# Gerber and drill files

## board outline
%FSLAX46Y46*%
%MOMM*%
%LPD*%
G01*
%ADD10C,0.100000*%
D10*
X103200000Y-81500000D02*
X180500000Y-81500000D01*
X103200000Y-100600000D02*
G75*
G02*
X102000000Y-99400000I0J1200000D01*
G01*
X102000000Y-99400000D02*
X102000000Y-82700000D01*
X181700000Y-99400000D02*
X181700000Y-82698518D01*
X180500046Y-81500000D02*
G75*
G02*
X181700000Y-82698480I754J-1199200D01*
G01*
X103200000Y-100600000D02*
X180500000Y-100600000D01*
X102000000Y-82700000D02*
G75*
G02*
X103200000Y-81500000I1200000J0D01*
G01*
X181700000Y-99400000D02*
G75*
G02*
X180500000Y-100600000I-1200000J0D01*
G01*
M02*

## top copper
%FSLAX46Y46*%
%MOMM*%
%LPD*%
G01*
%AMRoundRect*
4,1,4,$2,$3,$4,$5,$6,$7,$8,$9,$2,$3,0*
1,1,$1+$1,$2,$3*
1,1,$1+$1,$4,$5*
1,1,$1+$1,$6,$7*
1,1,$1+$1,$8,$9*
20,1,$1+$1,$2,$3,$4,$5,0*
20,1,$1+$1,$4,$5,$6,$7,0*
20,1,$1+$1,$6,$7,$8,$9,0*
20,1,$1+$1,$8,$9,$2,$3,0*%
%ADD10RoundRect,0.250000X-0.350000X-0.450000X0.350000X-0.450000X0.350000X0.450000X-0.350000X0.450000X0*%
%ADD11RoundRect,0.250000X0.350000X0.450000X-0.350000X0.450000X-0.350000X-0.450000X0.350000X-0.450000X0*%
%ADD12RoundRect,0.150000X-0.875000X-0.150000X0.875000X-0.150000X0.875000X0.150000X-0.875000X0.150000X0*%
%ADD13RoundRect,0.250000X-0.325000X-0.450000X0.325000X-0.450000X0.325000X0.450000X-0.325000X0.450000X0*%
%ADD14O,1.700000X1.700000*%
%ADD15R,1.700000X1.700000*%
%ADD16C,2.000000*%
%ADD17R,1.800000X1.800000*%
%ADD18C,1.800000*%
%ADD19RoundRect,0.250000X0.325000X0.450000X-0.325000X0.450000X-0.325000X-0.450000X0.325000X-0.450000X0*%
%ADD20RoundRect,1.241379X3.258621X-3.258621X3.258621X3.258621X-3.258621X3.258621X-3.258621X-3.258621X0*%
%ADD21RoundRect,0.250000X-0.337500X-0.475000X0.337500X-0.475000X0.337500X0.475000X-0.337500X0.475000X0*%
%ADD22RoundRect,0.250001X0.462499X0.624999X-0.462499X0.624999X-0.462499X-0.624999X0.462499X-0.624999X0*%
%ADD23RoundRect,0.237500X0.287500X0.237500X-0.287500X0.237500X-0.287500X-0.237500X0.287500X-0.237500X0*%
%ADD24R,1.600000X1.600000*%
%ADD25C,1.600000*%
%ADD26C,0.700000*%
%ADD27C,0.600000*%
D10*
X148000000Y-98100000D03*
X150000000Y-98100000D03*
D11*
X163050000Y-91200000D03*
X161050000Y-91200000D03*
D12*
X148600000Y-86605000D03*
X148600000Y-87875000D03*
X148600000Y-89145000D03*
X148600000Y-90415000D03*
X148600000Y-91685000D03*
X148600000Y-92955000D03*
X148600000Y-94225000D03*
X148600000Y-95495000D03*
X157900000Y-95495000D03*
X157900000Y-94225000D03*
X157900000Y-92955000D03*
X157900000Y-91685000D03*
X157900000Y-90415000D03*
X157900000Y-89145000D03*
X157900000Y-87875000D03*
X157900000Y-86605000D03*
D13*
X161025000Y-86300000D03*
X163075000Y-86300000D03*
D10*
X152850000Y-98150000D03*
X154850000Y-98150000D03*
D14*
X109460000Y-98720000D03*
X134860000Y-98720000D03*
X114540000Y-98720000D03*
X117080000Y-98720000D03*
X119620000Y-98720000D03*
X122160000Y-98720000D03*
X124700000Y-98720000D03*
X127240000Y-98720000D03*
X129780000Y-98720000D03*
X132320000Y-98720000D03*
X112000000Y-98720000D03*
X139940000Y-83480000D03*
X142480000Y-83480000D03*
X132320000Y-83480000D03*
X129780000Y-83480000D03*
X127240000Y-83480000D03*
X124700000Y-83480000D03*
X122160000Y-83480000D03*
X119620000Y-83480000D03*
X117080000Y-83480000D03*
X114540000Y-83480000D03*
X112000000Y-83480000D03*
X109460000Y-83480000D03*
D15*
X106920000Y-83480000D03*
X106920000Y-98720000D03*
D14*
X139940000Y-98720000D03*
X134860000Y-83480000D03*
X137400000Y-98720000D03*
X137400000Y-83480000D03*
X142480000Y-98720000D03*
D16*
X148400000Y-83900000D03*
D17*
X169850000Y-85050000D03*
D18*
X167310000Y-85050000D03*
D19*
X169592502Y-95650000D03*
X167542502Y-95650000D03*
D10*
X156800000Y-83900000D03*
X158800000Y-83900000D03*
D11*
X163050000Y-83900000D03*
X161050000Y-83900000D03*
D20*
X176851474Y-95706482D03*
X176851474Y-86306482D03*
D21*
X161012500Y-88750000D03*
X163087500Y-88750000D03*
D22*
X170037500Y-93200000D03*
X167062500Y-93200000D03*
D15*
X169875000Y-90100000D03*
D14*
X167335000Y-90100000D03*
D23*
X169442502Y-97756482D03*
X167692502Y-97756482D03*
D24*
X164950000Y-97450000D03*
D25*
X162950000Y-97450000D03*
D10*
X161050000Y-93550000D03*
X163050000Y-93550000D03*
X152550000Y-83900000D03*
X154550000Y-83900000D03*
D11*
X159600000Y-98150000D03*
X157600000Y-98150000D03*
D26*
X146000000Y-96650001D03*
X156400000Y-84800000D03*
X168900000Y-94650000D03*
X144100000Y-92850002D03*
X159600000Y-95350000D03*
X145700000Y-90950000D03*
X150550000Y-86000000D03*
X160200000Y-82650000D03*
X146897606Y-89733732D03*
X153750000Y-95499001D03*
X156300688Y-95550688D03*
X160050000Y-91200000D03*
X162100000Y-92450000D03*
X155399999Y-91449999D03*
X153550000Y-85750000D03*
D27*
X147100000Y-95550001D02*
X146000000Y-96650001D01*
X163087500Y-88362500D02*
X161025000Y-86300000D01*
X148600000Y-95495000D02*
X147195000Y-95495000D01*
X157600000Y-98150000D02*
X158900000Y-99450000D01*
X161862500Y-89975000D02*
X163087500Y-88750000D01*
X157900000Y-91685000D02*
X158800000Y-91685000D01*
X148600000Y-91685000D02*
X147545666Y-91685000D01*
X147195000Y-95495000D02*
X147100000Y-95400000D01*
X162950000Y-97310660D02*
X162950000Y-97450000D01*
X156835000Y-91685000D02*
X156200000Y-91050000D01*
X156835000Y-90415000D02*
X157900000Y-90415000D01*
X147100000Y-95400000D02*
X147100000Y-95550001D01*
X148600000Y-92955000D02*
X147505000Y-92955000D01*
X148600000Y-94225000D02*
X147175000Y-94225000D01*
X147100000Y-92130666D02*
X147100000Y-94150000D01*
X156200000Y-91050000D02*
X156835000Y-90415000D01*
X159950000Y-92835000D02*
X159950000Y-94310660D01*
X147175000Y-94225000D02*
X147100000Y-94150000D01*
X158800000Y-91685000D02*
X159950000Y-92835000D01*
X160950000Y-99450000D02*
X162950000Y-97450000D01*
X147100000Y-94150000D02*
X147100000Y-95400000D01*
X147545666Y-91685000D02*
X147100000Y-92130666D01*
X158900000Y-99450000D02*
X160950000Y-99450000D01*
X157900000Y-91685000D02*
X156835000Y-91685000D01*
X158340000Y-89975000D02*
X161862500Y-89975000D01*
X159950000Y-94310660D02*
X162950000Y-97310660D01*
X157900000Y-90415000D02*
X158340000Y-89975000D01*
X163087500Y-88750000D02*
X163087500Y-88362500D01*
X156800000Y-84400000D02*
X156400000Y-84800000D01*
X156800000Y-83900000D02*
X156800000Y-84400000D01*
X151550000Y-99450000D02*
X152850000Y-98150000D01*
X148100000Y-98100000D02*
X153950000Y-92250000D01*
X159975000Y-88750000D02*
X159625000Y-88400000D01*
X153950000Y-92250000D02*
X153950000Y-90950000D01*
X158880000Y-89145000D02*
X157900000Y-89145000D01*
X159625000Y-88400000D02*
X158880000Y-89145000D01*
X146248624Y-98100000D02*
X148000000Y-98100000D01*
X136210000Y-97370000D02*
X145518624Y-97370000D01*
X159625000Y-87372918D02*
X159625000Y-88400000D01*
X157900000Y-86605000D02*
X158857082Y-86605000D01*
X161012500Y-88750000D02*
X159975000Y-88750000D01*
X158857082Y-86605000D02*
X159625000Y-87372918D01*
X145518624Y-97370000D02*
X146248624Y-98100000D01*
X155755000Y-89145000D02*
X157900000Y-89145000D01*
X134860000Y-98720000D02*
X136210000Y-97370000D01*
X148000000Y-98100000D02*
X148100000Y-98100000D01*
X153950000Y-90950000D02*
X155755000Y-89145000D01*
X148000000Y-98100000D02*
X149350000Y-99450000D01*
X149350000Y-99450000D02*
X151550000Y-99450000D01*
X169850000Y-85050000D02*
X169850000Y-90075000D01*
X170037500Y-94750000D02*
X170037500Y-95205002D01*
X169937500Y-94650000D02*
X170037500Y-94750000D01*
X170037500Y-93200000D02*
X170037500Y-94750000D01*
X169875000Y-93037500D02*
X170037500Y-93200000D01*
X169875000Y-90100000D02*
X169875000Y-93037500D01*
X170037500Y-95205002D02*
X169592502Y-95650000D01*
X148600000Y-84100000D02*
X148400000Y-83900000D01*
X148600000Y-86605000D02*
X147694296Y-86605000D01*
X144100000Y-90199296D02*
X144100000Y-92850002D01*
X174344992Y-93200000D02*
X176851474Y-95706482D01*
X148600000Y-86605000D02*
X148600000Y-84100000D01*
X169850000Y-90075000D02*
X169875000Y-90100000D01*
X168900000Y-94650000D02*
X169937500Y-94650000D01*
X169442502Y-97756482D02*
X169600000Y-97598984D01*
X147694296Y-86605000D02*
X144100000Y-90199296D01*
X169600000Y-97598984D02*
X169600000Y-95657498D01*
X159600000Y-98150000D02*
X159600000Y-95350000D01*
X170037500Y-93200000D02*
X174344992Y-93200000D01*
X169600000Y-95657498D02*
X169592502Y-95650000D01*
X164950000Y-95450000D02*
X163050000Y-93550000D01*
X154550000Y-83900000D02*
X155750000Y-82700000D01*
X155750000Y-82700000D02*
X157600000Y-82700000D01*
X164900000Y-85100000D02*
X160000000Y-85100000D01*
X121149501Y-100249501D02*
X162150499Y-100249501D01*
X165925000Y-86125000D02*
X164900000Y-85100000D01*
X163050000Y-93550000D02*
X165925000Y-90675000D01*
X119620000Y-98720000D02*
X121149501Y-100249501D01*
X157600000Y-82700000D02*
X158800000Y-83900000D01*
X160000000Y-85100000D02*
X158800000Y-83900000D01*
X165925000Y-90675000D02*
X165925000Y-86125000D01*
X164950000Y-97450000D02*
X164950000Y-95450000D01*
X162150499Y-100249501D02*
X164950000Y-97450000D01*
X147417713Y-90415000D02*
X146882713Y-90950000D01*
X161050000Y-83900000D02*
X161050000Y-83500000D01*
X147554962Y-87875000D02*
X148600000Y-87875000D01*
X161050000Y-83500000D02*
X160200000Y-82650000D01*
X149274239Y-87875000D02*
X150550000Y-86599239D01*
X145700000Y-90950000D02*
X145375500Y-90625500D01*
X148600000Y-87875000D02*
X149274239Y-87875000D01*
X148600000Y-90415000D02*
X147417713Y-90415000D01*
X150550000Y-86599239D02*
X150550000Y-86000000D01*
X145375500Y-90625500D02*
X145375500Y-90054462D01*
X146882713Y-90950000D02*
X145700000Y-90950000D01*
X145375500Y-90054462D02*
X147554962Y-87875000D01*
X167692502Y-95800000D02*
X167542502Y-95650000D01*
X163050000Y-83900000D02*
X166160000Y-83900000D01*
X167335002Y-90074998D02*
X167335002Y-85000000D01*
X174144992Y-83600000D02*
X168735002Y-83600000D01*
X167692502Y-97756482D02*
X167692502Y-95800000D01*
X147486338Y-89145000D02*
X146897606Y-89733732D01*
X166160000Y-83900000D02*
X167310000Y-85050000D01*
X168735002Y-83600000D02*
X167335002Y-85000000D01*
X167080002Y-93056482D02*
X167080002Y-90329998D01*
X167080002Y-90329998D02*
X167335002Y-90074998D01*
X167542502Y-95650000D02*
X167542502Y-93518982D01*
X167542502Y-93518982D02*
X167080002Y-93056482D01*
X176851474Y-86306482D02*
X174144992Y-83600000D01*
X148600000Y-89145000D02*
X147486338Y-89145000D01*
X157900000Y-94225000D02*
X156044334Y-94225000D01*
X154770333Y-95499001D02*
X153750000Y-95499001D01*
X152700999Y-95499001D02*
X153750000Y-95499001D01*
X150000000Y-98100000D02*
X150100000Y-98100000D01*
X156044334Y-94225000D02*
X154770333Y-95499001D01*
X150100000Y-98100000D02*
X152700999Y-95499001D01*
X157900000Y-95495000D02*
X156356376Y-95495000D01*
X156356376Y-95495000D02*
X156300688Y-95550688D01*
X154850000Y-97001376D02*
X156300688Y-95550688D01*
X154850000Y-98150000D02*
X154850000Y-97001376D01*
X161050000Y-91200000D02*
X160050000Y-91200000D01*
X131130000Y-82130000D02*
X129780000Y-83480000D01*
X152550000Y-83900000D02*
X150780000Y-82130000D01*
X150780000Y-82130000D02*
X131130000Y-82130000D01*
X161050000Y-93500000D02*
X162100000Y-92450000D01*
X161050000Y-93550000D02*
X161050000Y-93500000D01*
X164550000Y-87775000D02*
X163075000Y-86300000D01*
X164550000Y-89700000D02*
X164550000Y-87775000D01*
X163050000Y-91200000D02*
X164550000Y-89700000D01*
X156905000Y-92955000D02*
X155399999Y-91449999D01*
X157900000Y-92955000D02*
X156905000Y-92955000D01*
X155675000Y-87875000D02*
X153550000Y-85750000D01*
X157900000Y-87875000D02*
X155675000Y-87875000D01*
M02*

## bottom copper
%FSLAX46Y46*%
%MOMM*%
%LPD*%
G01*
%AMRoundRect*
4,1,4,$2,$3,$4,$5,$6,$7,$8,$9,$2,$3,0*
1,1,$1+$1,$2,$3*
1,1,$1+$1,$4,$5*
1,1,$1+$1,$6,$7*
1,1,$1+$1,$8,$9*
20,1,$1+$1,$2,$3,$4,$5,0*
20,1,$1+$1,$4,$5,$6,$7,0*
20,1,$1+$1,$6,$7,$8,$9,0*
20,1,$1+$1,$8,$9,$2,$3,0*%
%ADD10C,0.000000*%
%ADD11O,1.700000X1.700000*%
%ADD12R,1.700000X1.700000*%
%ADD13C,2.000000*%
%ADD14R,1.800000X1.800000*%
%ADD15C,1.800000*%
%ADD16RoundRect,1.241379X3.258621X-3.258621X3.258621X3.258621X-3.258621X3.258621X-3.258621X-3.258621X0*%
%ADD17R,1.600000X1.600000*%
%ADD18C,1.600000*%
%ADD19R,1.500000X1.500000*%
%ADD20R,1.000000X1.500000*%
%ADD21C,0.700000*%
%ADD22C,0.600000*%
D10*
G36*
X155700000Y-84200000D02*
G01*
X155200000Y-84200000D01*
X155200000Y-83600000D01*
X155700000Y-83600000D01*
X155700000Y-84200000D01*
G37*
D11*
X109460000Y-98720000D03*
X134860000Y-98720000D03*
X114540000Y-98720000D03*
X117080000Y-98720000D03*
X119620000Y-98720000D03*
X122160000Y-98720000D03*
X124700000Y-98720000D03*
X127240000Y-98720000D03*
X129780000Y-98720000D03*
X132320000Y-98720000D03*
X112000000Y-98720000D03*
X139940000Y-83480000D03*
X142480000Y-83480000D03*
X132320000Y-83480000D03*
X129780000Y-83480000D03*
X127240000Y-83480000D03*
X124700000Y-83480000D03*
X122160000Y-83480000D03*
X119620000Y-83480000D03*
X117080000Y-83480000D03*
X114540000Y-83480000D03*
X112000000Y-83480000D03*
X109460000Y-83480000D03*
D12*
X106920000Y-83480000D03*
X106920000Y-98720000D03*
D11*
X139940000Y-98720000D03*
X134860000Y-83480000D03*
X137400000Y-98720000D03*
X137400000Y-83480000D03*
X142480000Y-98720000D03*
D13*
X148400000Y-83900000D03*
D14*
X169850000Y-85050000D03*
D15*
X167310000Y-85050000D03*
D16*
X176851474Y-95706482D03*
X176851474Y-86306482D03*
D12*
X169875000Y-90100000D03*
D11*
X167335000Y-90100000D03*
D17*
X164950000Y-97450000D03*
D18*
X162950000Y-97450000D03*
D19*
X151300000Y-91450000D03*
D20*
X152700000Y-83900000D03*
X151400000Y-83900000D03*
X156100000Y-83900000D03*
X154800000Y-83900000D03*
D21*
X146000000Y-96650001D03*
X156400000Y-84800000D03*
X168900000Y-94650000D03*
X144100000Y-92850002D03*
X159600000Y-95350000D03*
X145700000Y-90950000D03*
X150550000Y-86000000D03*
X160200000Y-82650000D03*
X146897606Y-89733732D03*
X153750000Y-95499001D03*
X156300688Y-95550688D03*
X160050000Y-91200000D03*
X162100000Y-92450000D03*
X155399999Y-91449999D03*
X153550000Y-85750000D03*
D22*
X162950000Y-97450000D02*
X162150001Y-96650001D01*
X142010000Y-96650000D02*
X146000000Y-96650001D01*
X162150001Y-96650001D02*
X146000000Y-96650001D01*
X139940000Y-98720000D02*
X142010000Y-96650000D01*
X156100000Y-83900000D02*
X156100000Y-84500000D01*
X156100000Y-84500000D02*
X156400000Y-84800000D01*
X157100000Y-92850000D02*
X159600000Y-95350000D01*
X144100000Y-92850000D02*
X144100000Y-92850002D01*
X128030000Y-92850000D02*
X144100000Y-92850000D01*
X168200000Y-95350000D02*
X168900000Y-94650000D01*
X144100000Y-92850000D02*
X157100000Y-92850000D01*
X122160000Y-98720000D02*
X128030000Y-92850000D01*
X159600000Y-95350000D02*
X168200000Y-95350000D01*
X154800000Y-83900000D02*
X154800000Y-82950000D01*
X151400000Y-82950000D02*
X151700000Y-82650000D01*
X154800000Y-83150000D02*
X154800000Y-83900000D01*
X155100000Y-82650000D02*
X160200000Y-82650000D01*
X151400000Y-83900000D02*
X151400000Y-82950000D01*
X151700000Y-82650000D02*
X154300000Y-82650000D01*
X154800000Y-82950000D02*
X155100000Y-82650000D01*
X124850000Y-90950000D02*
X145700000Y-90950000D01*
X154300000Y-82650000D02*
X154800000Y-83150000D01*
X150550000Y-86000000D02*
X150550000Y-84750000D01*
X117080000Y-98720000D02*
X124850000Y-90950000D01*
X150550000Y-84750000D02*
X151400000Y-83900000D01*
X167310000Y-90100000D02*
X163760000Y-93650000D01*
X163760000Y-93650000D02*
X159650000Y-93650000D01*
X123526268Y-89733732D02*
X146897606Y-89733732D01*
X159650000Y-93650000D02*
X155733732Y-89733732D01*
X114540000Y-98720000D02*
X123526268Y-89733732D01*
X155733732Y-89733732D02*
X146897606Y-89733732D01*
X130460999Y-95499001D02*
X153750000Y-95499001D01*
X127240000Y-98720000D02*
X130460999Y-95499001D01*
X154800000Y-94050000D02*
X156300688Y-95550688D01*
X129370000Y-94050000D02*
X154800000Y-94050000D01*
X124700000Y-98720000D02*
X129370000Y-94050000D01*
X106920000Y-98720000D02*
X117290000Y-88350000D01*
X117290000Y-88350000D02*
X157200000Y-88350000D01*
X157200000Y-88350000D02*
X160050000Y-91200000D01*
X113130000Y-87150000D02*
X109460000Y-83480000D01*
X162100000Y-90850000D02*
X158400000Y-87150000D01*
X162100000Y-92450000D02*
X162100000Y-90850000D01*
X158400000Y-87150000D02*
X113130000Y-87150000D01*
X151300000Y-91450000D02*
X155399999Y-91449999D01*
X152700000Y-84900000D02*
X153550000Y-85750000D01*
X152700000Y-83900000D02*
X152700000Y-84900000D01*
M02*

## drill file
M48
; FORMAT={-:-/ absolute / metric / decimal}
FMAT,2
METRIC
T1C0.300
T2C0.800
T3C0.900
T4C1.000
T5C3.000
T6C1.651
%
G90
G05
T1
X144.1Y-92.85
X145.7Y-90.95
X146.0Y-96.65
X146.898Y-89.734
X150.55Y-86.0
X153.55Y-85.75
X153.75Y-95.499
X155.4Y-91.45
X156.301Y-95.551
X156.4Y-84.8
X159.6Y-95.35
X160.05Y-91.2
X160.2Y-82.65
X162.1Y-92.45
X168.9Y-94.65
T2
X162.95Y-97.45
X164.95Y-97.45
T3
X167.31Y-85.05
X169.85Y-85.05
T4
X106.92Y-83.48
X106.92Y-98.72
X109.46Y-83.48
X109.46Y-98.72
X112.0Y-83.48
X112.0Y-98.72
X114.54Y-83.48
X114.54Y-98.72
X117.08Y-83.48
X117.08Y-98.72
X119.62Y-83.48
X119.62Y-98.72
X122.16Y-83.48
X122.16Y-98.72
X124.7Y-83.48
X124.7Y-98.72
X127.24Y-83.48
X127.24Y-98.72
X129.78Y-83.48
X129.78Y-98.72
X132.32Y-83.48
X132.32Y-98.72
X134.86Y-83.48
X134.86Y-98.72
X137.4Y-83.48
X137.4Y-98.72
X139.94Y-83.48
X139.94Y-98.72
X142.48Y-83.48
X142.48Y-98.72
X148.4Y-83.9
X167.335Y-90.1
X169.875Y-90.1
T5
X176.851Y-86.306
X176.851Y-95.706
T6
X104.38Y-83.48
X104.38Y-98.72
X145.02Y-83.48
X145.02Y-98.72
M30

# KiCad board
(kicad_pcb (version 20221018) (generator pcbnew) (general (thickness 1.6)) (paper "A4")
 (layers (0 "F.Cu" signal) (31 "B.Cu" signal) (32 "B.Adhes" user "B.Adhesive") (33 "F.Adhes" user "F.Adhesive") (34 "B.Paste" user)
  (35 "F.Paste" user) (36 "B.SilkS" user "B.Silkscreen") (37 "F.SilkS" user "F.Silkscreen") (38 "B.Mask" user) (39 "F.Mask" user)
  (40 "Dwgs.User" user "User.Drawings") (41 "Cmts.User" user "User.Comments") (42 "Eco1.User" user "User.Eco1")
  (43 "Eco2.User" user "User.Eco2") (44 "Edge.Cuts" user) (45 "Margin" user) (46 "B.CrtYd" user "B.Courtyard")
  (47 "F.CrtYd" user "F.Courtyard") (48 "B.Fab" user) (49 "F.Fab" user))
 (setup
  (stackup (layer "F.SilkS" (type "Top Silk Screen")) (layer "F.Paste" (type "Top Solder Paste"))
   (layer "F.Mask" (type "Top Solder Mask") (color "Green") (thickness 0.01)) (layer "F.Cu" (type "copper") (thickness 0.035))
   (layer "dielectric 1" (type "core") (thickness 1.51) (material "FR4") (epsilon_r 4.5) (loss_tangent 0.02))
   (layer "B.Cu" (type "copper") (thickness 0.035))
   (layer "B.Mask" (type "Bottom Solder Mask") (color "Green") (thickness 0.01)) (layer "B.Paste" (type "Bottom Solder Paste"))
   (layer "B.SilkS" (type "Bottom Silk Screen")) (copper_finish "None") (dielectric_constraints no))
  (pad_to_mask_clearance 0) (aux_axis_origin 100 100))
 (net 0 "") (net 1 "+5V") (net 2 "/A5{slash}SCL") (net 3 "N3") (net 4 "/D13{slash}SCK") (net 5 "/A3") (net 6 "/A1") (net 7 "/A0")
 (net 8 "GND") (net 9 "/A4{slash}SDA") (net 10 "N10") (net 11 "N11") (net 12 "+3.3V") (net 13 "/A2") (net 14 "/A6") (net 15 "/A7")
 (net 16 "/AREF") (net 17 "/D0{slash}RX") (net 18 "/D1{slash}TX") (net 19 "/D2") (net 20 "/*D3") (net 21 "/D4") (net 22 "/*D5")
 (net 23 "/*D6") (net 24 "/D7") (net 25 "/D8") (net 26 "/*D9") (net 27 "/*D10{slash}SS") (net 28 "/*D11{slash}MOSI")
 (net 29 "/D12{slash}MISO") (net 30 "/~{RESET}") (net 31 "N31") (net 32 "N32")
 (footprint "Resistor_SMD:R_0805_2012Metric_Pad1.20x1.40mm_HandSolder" (layer "F.Cu") (at 149 98.1)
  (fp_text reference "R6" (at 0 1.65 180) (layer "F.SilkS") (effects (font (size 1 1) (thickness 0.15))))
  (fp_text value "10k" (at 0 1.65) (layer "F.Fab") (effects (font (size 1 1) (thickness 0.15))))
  (pad "1" smd roundrect (at -1 0) (size 1.2 1.4) (layers "F.Cu" "F.Paste" "F.Mask") (roundrect_rratio 0.208333) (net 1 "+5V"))
  (pad "2" smd roundrect (at 1 0) (size 1.2 1.4) (layers "F.Cu" "F.Paste" "F.Mask") (roundrect_rratio 0.208333) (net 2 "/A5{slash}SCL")))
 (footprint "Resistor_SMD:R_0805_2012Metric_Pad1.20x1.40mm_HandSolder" (layer "F.Cu") (at 162.05 91.2 180)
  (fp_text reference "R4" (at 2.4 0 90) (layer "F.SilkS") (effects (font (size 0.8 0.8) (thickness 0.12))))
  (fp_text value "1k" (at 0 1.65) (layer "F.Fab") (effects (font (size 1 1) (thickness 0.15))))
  (pad "1" smd roundrect (at -1 0 180) (size 1.2 1.4) (layers "F.Cu" "F.Paste" "F.Mask") (roundrect_rratio 0.2083333333) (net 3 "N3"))
  (pad "2" smd roundrect (at 1 0 180) (size 1.2 1.4) (layers "F.Cu" "F.Paste" "F.Mask") (roundrect_rratio 0.2083333333)
   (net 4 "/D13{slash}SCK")))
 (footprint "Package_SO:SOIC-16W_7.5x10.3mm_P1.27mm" (layer "F.Cu") (at 153.25 91.05)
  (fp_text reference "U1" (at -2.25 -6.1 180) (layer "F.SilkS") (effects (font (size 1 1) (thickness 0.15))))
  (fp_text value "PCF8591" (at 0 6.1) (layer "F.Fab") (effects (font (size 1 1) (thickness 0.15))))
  (pad "1" smd roundrect (at -4.65 -4.445) (size 2.05 0.6) (layers "F.Cu" "F.Paste" "F.Mask") (roundrect_rratio 0.25) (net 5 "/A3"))
  (pad "2" smd roundrect (at -4.65 -3.175) (size 2.05 0.6) (layers "F.Cu" "F.Paste" "F.Mask") (roundrect_rratio 0.25) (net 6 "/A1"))
  (pad "3" smd roundrect (at -4.65 -1.905) (size 2.05 0.6) (layers "F.Cu" "F.Paste" "F.Mask") (roundrect_rratio 0.25) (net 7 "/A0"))
  (pad "4" smd roundrect (at -4.65 -0.635) (size 2.05 0.6) (layers "F.Cu" "F.Paste" "F.Mask") (roundrect_rratio 0.25) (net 6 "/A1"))
  (pad "5" smd roundrect (at -4.65 0.635) (size 2.05 0.6) (layers "F.Cu" "F.Paste" "F.Mask") (roundrect_rratio 0.25) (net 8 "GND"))
  (pad "6" smd roundrect (at -4.65 1.905) (size 2.05 0.6) (layers "F.Cu" "F.Paste" "F.Mask") (roundrect_rratio 0.25) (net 8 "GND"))
  (pad "7" smd roundrect (at -4.65 3.175) (size 2.05 0.6) (layers "F.Cu" "F.Paste" "F.Mask") (roundrect_rratio 0.25) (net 8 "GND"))
  (pad "8" smd roundrect (at -4.65 4.445) (size 2.05 0.6) (layers "F.Cu" "F.Paste" "F.Mask") (roundrect_rratio 0.25) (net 8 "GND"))
  (pad "9" smd roundrect (at 4.65 4.445) (size 2.05 0.6) (layers "F.Cu" "F.Paste" "F.Mask") (roundrect_rratio 0.25) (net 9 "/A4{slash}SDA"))
  (pad "10" smd roundrect (at 4.65 3.175) (size 2.05 0.6) (layers "F.Cu" "F.Paste" "F.Mask") (roundrect_rratio 0.25) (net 2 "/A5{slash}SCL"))
  (pad "11" smd roundrect (at 4.65 1.905) (size 2.05 0.6) (layers "F.Cu" "F.Paste" "F.Mask") (roundrect_rratio 0.25) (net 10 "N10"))
  (pad "12" smd roundrect (at 4.65 0.635) (size 2.05 0.6) (layers "F.Cu" "F.Paste" "F.Mask") (roundrect_rratio 0.25) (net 8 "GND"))
  (pad "13" smd roundrect (at 4.65 -0.635) (size 2.05 0.6) (layers "F.Cu" "F.Paste" "F.Mask") (roundrect_rratio 0.25) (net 8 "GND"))
  (pad "14" smd roundrect (at 4.65 -1.905) (size 2.05 0.6) (layers "F.Cu" "F.Paste" "F.Mask") (roundrect_rratio 0.25) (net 1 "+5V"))
  (pad "15" smd roundrect (at 4.65 -3.175) (size 2.05 0.6) (layers "F.Cu" "F.Paste" "F.Mask") (roundrect_rratio 0.25) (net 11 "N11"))
  (pad "16" smd roundrect (at 4.65 -4.445) (size 2.05 0.6) (layers "F.Cu" "F.Paste" "F.Mask") (roundrect_rratio 0.25) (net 1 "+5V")))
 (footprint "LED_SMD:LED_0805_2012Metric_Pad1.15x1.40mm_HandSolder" (layer "F.Cu") (at 162.05 86.3)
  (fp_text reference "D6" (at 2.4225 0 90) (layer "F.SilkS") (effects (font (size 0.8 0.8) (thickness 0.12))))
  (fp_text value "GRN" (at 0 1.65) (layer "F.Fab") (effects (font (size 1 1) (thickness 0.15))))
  (pad "1" smd roundrect (at -1.025 0) (size 1.15 1.4) (layers "F.Cu" "F.Paste" "F.Mask") (roundrect_rratio 0.2173913043) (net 8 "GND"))
  (pad "2" smd roundrect (at 1.025 0) (size 1.15 1.4) (layers "F.Cu" "F.Paste" "F.Mask") (roundrect_rratio 0.2173913043) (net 3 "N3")))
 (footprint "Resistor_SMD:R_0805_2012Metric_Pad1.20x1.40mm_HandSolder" (layer "F.Cu") (at 153.85 98.15)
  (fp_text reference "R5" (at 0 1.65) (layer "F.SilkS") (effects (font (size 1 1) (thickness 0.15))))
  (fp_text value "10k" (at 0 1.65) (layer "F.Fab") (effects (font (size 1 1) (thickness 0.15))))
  (pad "1" smd roundrect (at -1 0) (size 1.2 1.4) (layers "F.Cu" "F.Paste" "F.Mask") (roundrect_rratio 0.208333) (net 1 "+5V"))
  (pad "2" smd roundrect (at 1 0) (size 1.2 1.4) (layers "F.Cu" "F.Paste" "F.Mask") (roundrect_rratio 0.208333) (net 9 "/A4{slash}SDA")))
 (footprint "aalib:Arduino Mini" (layer "F.Cu") (at 124.7 91.1 90)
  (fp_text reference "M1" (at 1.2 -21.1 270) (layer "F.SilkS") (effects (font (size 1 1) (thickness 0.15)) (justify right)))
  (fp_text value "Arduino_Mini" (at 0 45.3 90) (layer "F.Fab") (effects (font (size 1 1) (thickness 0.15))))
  (pad "" np_thru_hole circle (at -7.62 -20.32 90) (size 1.651 1.651) (drill 1.651) (layers "*.Mask"))
  (pad "" np_thru_hole circle (at -7.62 20.32 90) (size 1.651 1.651) (drill 1.651) (layers "*.Mask"))
  (pad "" np_thru_hole circle (at 7.62 -20.32 90) (size 1.651 1.651) (drill 1.651) (layers "*.Mask"))
  (pad "" np_thru_hole circle (at 7.62 20.32 90) (size 1.651 1.651) (drill 1.651) (layers "*.Mask"))
  (pad "3V3" thru_hole oval (at -7.62 -15.24 90) (size 1.7 1.7) (drill 1) (layers "*.Cu" "*.Mask") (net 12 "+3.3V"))
  (pad "5V" thru_hole oval (at -7.62 10.16 90) (size 1.7 1.7) (drill 1) (layers "*.Cu" "*.Mask") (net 1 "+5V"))
  (pad "A0" thru_hole oval (at -7.62 -10.16 90) (size 1.7 1.7) (drill 1) (layers "*.Cu" "*.Mask") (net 7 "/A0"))
  (pad "A1" thru_hole oval (at -7.62 -7.62 90) (size 1.7 1.7) (drill 1) (layers "*.Cu" "*.Mask") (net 6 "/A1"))
  (pad "A2" thru_hole oval (at -7.62 -5.08 90) (size 1.7 1.7) (drill 1) (layers "*.Cu" "*.Mask") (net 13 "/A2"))
  (pad "A3" thru_hole oval (at -7.62 -2.54 90) (size 1.7 1.7) (drill 1) (layers "*.Cu" "*.Mask") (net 5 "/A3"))
  (pad "A4" thru_hole oval (at -7.62 0 90) (size 1.7 1.7) (drill 1) (layers "*.Cu" "*.Mask") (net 9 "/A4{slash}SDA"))
  (pad "A5" thru_hole oval (at -7.62 2.54 90) (size 1.7 1.7) (drill 1) (layers "*.Cu" "*.Mask") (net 2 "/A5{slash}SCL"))
  (pad "A6" thru_hole oval (at -7.62 5.08 90) (size 1.7 1.7) (drill 1) (layers "*.Cu" "*.Mask") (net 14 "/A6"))
  (pad "A7" thru_hole oval (at -7.62 7.62 90) (size 1.7 1.7) (drill 1) (layers "*.Cu" "*.Mask") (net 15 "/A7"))
  (pad "AREF" thru_hole oval (at -7.62 -12.7 90) (size 1.7 1.7) (drill 1) (layers "*.Cu" "*.Mask") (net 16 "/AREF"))
  (pad "D0/RX" thru_hole oval (at 7.62 15.24 90) (size 1.7 1.7) (drill 1) (layers "*.Cu" "*.Mask") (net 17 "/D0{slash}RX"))
  (pad "D1/TX" thru_hole oval (at 7.62 17.78 90) (size 1.7 1.7) (drill 1) (layers "*.Cu" "*.Mask") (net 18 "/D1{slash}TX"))
  (pad "D2" thru_hole oval (at 7.62 7.62 90) (size 1.7 1.7) (drill 1) (layers "*.Cu" "*.Mask") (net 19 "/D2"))
  (pad "D3" thru_hole oval (at 7.62 5.08 90) (size 1.7 1.7) (drill 1) (layers "*.Cu" "*.Mask") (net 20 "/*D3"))
  (pad "D4" thru_hole oval (at 7.62 2.54 90) (size 1.7 1.7) (drill 1) (layers "*.Cu" "*.Mask") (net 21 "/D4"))
  (pad "D5" thru_hole oval (at 7.62 0 90) (size 1.7 1.7) (drill 1) (layers "*.Cu" "*.Mask") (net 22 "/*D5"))
  (pad "D6" thru_hole oval (at 7.62 -2.54 90) (size 1.7 1.7) (drill 1) (layers "*.Cu" "*.Mask") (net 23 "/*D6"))
  (pad "D7" thru_hole oval (at 7.62 -5.08 90) (size 1.7 1.7) (drill 1) (layers "*.Cu" "*.Mask") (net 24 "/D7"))
  (pad "D8" thru_hole oval (at 7.62 -7.62 90) (size 1.7 1.7) (drill 1) (layers "*.Cu" "*.Mask") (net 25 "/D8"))
  (pad "D9" thru_hole oval (at 7.62 -10.16 90) (size 1.7 1.7) (drill 1) (layers "*.Cu" "*.Mask") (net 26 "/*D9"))
  (pad "D10" thru_hole oval (at 7.62 -12.7 90) (size 1.7 1.7) (drill 1) (layers "*.Cu" "*.Mask") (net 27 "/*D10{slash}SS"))
  (pad "D11" thru_hole oval (at 7.62 -15.24 90) (size 1.7 1.7) (drill 1) (layers "*.Cu" "*.Mask") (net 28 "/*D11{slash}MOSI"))
  (pad "D12" thru_hole rect (at 7.62 -17.78 90) (size 1.7 1.7) (drill 1) (layers "*.Cu" "*.Mask") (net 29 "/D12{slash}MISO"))
  (pad "D13" thru_hole rect (at -7.62 -17.78 90) (size 1.7 1.7) (drill 1) (layers "*.Cu" "*.Mask") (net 4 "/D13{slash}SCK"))
  (pad "GND" thru_hole oval (at -7.62 15.24 90) (size 1.7 1.7) (drill 1) (layers "*.Cu" "*.Mask") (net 8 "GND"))
  (pad "GND" thru_hole oval (at 7.62 10.16 90) (size 1.7 1.7) (drill 1) (layers "*.Cu" "*.Mask") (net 8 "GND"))
  (pad "RESET" thru_hole oval (at -7.62 12.7 90) (size 1.7 1.7) (drill 1) (layers "*.Cu" "*.Mask") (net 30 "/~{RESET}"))
  (pad "RESET" thru_hole oval (at 7.62 12.7 90) (size 1.7 1.7) (drill 1) (layers "*.Cu" "*.Mask") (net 30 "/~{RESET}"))
  (pad "VIN" thru_hole oval (at -7.62 17.78 90) (size 1.7 1.7) (drill 1) (layers "*.Cu" "*.Mask") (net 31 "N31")))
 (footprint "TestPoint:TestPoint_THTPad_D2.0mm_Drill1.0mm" (layer "F.Cu") (at 148.4 83.9)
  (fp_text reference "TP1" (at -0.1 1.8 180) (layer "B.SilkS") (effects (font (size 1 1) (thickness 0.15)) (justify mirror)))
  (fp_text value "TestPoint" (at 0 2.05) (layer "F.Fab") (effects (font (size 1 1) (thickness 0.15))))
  (pad "1" thru_hole circle (at 0 0) (size 2 2) (drill 1) (layers "*.Cu" "*.Mask") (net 5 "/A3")))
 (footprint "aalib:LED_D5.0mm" (layer "F.Cu") (at 169.85 85.05 180)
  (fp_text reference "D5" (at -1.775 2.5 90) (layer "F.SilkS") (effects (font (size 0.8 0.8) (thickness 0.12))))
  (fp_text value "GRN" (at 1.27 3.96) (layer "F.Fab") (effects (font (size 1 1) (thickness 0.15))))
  (pad "1" thru_hole rect (at 0 0 180) (size 1.8 1.8) (drill 0.9) (layers "*.Cu" "*.Mask") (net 5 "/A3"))
  (pad "2" thru_hole circle (at 2.54 0 180) (size 1.8 1.8) (drill 0.9) (layers "*.Cu" "*.Mask") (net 7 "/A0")))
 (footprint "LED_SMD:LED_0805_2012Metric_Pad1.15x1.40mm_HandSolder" (layer "F.Cu") (at 168.567502 95.65 180)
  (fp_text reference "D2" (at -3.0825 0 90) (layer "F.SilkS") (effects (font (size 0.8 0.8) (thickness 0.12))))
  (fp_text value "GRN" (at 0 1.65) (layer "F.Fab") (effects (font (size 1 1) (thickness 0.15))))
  (pad "1" smd roundrect (at -1.025 0 180) (size 1.15 1.4) (layers "F.Cu" "F.Paste" "F.Mask") (roundrect_rratio 0.217391) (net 5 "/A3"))
  (pad "2" smd roundrect (at 1.025 0 180) (size 1.15 1.4) (layers "F.Cu" "F.Paste" "F.Mask") (roundrect_rratio 0.217391) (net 7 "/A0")))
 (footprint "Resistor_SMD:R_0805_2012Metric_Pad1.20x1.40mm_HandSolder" (layer "F.Cu") (at 157.8 83.9)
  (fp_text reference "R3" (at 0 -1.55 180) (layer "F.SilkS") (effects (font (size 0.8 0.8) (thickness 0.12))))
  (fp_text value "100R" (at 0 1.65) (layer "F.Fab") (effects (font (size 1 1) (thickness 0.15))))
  (pad "1" smd roundrect (at -1 0) (size 1.2 1.4) (layers "F.Cu" "F.Paste" "F.Mask") (roundrect_rratio 0.2083333333) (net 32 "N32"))
  (pad "2" smd roundrect (at 1 0) (size 1.2 1.4) (layers "F.Cu" "F.Paste" "F.Mask") (roundrect_rratio 0.2083333333) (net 13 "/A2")))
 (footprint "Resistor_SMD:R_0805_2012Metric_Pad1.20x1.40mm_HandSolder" (layer "F.Cu") (at 162.05 83.9 180)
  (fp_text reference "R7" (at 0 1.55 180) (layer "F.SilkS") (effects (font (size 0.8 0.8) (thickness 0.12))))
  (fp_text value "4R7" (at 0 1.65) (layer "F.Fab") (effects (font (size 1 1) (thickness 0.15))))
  (pad "1" smd roundrect (at -1 0 180) (size 1.2 1.4) (layers "F.Cu" "F.Paste" "F.Mask") (roundrect_rratio 0.208333) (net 7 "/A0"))
  (pad "2" smd roundrect (at 1 0 180) (size 1.2 1.4) (layers "F.Cu" "F.Paste" "F.Mask") (roundrect_rratio 0.208333) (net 6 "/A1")))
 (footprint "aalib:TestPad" (layer "F.Cu") (at 176.851474 91.006482 90)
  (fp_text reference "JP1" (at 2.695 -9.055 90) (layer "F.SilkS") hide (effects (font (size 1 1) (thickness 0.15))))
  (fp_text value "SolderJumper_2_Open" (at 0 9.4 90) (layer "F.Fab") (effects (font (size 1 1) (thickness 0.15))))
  (pad "1" thru_hole roundrect (at -4.7 0 90) (size 9 9) (drill 3) (layers "*.Cu" "*.Mask") (roundrect_rratio 0.137931) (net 5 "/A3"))
  (pad "2" thru_hole roundrect (at 4.7 0 90) (size 9 9) (drill 3) (layers "*.Cu" "*.Mask") (roundrect_rratio 0.137931) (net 7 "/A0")))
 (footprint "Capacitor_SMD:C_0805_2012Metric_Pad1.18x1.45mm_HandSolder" (layer "F.Cu") (at 162.05 88.75)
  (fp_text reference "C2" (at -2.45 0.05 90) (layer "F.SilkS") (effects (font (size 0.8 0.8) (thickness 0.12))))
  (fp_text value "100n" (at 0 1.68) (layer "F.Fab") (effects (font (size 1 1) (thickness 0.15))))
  (pad "1" smd roundrect (at -1.0375 0) (size 1.175 1.45) (layers "F.Cu" "F.Paste" "F.Mask") (roundrect_rratio 0.212766) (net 1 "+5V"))
  (pad "2" smd roundrect (at 1.0375 0) (size 1.175 1.45) (layers "F.Cu" "F.Paste" "F.Mask") (roundrect_rratio 0.212766) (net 8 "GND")))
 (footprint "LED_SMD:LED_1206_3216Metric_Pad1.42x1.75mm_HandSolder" (layer "F.Cu") (at 168.55 93.2 180)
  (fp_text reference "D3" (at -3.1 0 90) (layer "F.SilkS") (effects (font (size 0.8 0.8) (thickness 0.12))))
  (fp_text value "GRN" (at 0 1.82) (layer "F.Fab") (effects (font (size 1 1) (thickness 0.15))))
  (pad "1" smd roundrect (at -1.4875 0 180) (size 1.425 1.75) (layers "F.Cu" "F.Paste" "F.Mask") (roundrect_rratio 0.175439) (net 5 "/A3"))
  (pad "2" smd roundrect (at 1.4875 0 180) (size 1.425 1.75) (layers "F.Cu" "F.Paste" "F.Mask") (roundrect_rratio 0.175439) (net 7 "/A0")))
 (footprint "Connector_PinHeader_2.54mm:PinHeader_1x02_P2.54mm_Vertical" (layer "F.Cu") (at 169.875 90.1 -90)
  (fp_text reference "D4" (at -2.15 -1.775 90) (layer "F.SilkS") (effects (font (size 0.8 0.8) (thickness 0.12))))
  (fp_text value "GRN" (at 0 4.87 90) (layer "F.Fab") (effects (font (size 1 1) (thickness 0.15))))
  (pad "1" thru_hole rect (at 0 0 270) (size 1.7 1.7) (drill 1) (layers "*.Cu" "*.Mask") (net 5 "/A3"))
  (pad "2" thru_hole oval (at 0 2.54 270) (size 1.7 1.7) (drill 1) (layers "*.Cu" "*.Mask") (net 7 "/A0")))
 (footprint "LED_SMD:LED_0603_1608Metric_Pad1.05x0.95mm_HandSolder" (layer "F.Cu") (at 168.567502 97.756482 180)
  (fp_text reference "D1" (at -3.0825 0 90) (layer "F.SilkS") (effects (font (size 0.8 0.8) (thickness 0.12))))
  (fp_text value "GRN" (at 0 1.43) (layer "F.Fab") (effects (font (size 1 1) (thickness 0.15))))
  (pad "1" smd roundrect (at -0.875 0 180) (size 1.05 0.95) (layers "F.Cu" "F.Paste" "F.Mask") (roundrect_rratio 0.25) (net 5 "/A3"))
  (pad "2" smd roundrect (at 0.875 0 180) (size 1.05 0.95) (layers "F.Cu" "F.Paste" "F.Mask") (roundrect_rratio 0.25) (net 7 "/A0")))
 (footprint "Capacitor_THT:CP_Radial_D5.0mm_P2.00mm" (layer "F.Cu") (at 164.95 97.45 180)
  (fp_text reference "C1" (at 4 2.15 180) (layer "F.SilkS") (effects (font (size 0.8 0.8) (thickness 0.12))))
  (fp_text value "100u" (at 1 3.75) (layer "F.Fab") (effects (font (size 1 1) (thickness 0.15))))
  (pad "1" thru_hole rect (at 0 0 180) (size 1.6 1.6) (drill 0.8) (layers "*.Cu" "*.Mask") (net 13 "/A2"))
  (pad "2" thru_hole circle (at 2 0 180) (size 1.6 1.6) (drill 0.8) (layers "*.Cu" "*.Mask") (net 8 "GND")))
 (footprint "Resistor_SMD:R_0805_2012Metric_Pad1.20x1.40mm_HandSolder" (layer "F.Cu") (at 162.05 93.55)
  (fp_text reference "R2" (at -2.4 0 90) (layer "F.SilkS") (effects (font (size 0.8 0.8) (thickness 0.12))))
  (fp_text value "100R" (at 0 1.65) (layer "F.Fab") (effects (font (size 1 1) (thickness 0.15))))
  (pad "1" smd roundrect (at -1 0) (size 1.2 1.4) (layers "F.Cu" "F.Paste" "F.Mask") (roundrect_rratio 0.2083333333)
   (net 28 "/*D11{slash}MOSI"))
  (pad "2" smd roundrect (at 1 0) (size 1.2 1.4) (layers "F.Cu" "F.Paste" "F.Mask") (roundrect_rratio 0.2083333333) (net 13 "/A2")))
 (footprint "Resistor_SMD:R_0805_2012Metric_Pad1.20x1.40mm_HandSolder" (layer "F.Cu") (at 153.55 83.9)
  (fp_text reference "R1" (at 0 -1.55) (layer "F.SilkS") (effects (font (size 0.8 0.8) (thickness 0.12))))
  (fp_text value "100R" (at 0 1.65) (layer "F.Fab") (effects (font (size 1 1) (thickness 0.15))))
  (pad "1" smd roundrect (at -1 0) (size 1.2 1.4) (layers "F.Cu" "F.Paste" "F.Mask") (roundrect_rratio 0.2083333333) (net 20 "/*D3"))
  (pad "2" smd roundrect (at 1 0) (size 1.2 1.4) (layers "F.Cu" "F.Paste" "F.Mask") (roundrect_rratio 0.2083333333) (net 13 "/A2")))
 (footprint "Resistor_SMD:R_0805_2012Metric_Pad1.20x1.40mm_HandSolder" (layer "F.Cu") (at 158.6 98.15 180)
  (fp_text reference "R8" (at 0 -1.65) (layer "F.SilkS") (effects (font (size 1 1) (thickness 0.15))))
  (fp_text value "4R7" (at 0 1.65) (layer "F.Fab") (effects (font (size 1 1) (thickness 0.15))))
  (pad "1" smd roundrect (at -1 0 180) (size 1.2 1.4) (layers "F.Cu" "F.Paste" "F.Mask") (roundrect_rratio 0.208333) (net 5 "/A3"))
  (pad "2" smd roundrect (at 1 0 180) (size 1.2 1.4) (layers "F.Cu" "F.Paste" "F.Mask") (roundrect_rratio 0.208333) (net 8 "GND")))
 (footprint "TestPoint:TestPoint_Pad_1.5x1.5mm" (layer "B.Cu") (at 151.3 91.45)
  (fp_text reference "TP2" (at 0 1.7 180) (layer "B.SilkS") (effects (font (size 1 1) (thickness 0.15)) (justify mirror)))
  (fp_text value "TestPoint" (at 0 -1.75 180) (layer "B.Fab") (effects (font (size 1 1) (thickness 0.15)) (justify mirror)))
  (pad "1" smd rect (at 0 0) (size 1.5 1.5) (layers "B.Cu" "B.Mask") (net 10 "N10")))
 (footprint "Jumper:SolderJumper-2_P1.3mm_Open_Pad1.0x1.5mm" (layer "B.Cu") (at 152.05 83.9 180)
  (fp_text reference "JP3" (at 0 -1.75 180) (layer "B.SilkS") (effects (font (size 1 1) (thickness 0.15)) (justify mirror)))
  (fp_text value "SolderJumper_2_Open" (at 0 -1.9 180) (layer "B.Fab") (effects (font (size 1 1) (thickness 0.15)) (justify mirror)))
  (pad "1" smd rect (at -0.65 0 180) (size 1 1.5) (layers "B.Cu" "B.Mask") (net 11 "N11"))
  (pad "2" smd rect (at 0.65 0 180) (size 1 1.5) (layers "B.Cu" "B.Mask") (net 6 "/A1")))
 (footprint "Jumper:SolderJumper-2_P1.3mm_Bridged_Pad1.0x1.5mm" (layer "B.Cu") (at 155.45 83.9 180) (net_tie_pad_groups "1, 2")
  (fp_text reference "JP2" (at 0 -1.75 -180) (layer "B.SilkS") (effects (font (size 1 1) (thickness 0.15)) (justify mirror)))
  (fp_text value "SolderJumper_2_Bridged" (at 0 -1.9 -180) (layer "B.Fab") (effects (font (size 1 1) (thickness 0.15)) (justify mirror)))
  (fp_poly (pts (xy -0.25 0.3) (xy 0.25 0.3) (xy 0.25 -0.3) (xy -0.25 -0.3)) (stroke (width 0) (type solid)) (fill solid) (layer "B.Cu"))
  (pad "1" smd rect (at -0.65 0 180) (size 1 1.5) (layers "B.Cu" "B.Mask") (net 32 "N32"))
  (pad "2" smd rect (at 0.65 0 180) (size 1 1.5) (layers "B.Cu" "B.Mask") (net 6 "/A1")))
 (gr_line (start 103.2 81.5) (end 180.5 81.5) (stroke (width 0.1) (type solid)) (layer "Edge.Cuts"))
 (gr_arc (start 103.2 100.6) (mid 102.351472 100.248528) (end 102 99.4) (stroke (width 0.1) (type solid)) (layer "Edge.Cuts"))
 (gr_line (start 102 99.4) (end 102 82.7) (stroke (width 0.1) (type solid)) (layer "Edge.Cuts"))
 (gr_line (start 181.7 99.4) (end 181.7 82.698518) (stroke (width 0.1) (type default)) (layer "Edge.Cuts"))
 (gr_arc (start 180.500046 81.5) (mid 181.348236 81.850721) (end 181.7 82.69848) (stroke (width 0.1) (type solid)) (layer "Edge.Cuts"))
 (gr_line (start 103.2 100.6) (end 180.5 100.6) (stroke (width 0.1) (type solid)) (layer "Edge.Cuts"))
 (gr_arc (start 102 82.7) (mid 102.351472 81.851472) (end 103.2 81.5) (stroke (width 0.1) (type solid)) (layer "Edge.Cuts"))
 (gr_arc (start 181.7 99.4) (mid 181.348528 100.248528) (end 180.5 100.6) (stroke (width 0.1) (type solid)) (layer "Edge.Cuts"))
 (segment (start 147.1 95.550001) (end 146 96.650001) (width 0.6) (layer "F.Cu") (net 8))
 (segment (start 163.0875 88.3625) (end 161.025 86.3) (width 0.6) (layer "F.Cu") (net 8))
 (segment (start 148.6 95.495) (end 147.195 95.495) (width 0.6) (layer "F.Cu") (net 8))
 (segment (start 157.6 98.15) (end 158.9 99.45) (width 0.6) (layer "F.Cu") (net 8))
 (segment (start 161.8625 89.975) (end 163.0875 88.75) (width 0.6) (layer "F.Cu") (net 8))
 (segment (start 157.9 91.685) (end 158.8 91.685) (width 0.6) (layer "F.Cu") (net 8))
 (segment (start 148.6 91.685) (end 147.545666 91.685) (width 0.6) (layer "F.Cu") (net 8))
 (segment (start 147.195 95.495) (end 147.1 95.4) (width 0.6) (layer "F.Cu") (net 8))
 (segment (start 162.95 97.31066) (end 162.95 97.45) (width 0.6) (layer "F.Cu") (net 8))
 (segment (start 156.835 91.685) (end 156.2 91.05) (width 0.6) (layer "F.Cu") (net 8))
 (segment (start 156.835 90.415) (end 157.9 90.415) (width 0.6) (layer "F.Cu") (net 8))
 (segment (start 147.1 95.4) (end 147.1 95.550001) (width 0.6) (layer "F.Cu") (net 8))
 (segment (start 148.6 92.955) (end 147.505 92.955) (width 0.6) (layer "F.Cu") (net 8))
 (segment (start 148.6 94.225) (end 147.175 94.225) (width 0.6) (layer "F.Cu") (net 8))
 (segment (start 147.1 92.130666) (end 147.1 94.15) (width 0.6) (layer "F.Cu") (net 8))
 (segment (start 156.2 91.05) (end 156.835 90.415) (width 0.6) (layer "F.Cu") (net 8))
 (segment (start 159.95 92.835) (end 159.95 94.31066) (width 0.6) (layer "F.Cu") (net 8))
 (segment (start 147.175 94.225) (end 147.1 94.15) (width 0.6) (layer "F.Cu") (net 8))
 (segment (start 158.8 91.685) (end 159.95 92.835) (width 0.6) (layer "F.Cu") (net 8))
 (segment (start 160.95 99.45) (end 162.95 97.45) (width 0.6) (layer "F.Cu") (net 8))
 (segment (start 147.1 94.15) (end 147.1 95.4) (width 0.6) (layer "F.Cu") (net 8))
 (segment (start 147.545666 91.685) (end 147.1 92.130666) (width 0.6) (layer "F.Cu") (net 8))
 (segment (start 158.9 99.45) (end 160.95 99.45) (width 0.6) (layer "F.Cu") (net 8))
 (segment (start 157.9 91.685) (end 156.835 91.685) (width 0.6) (layer "F.Cu") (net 8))
 (segment (start 158.34 89.975) (end 161.8625 89.975) (width 0.6) (layer "F.Cu") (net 8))
 (segment (start 159.95 94.31066) (end 162.95 97.31066) (width 0.6) (layer "F.Cu") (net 8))
 (segment (start 157.9 90.415) (end 158.34 89.975) (width 0.6) (layer "F.Cu") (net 8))
 (segment (start 163.0875 88.75) (end 163.0875 88.3625) (width 0.6) (layer "F.Cu") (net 8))
 (via (at 146 96.650001) (size 0.7) (drill 0.3) (layers "F.Cu" "B.Cu") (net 8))
 (segment (start 162.95 97.45) (end 162.150001 96.650001) (width 0.6) (layer "B.Cu") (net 8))
 (segment (start 142.01 96.65) (end 146 96.650001) (width 0.6) (layer "B.Cu") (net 8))
 (segment (start 162.150001 96.650001) (end 146 96.650001) (width 0.6) (layer "B.Cu") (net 8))
 (segment (start 139.94 98.72) (end 142.01 96.65) (width 0.6) (layer "B.Cu") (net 8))
 (segment (start 156.8 84.4) (end 156.4 84.8) (width 0.6) (layer "F.Cu") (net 32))
 (segment (start 156.8 83.9) (end 156.8 84.4) (width 0.6) (layer "F.Cu") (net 32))
 (via (at 156.4 84.8) (size 0.7) (drill 0.3) (layers "F.Cu" "B.Cu") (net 32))
 (segment (start 156.1 83.9) (end 156.1 84.5) (width 0.6) (layer "B.Cu") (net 32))
 (segment (start 156.1 84.5) (end 156.4 84.8) (width 0.6) (layer "B.Cu") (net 32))
 (segment (start 151.55 99.45) (end 152.85 98.15) (width 0.6) (layer "F.Cu") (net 1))
 (segment (start 148.1 98.1) (end 153.95 92.25) (width 0.6) (layer "F.Cu") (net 1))
 (segment (start 159.975 88.75) (end 159.625 88.4) (width 0.6) (layer "F.Cu") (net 1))
 (segment (start 153.95 92.25) (end 153.95 90.95) (width 0.6) (layer "F.Cu") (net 1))
 (segment (start 158.88 89.145) (end 157.9 89.145) (width 0.6) (layer "F.Cu") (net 1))
 (segment (start 159.625 88.4) (end 158.88 89.145) (width 0.6) (layer "F.Cu") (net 1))
 (segment (start 146.248624 98.1) (end 148 98.1) (width 0.6) (layer "F.Cu") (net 1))
 (segment (start 136.21 97.37) (end 145.518624 97.37) (width 0.6) (layer "F.Cu") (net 1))
 (segment (start 159.625 87.372918) (end 159.625 88.4) (width 0.6) (layer "F.Cu") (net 1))
 (segment (start 157.9 86.605) (end 158.857082 86.605) (width 0.6) (layer "F.Cu") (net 1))
 (segment (start 161.0125 88.75) (end 159.975 88.75) (width 0.6) (layer "F.Cu") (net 1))
 (segment (start 158.857082 86.605) (end 159.625 87.372918) (width 0.6) (layer "F.Cu") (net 1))
 (segment (start 145.518624 97.37) (end 146.248624 98.1) (width 0.6) (layer "F.Cu") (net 1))
 (segment (start 155.755 89.145) (end 157.9 89.145) (width 0.6) (layer "F.Cu") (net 1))
 (segment (start 134.86 98.72) (end 136.21 97.37) (width 0.6) (layer "F.Cu") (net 1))
 (segment (start 148 98.1) (end 148.1 98.1) (width 0.6) (layer "F.Cu") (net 1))
 (segment (start 153.95 90.95) (end 155.755 89.145) (width 0.6) (layer "F.Cu") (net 1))
 (segment (start 148 98.1) (end 149.35 99.45) (width 0.6) (layer "F.Cu") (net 1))
 (segment (start 149.35 99.45) (end 151.55 99.45) (width 0.6) (layer "F.Cu") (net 1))
 (segment (start 169.85 85.05) (end 169.85 90.075) (width 0.6) (layer "F.Cu") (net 5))
 (segment (start 170.0375 94.75) (end 170.0375 95.205002) (width 0.6) (layer "F.Cu") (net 5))
 (segment (start 169.9375 94.65) (end 170.0375 94.75) (width 0.6) (layer "F.Cu") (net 5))
 (segment (start 170.0375 93.2) (end 170.0375 94.75) (width 0.6) (layer "F.Cu") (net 5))
 (segment (start 169.875 93.0375) (end 170.0375 93.2) (width 0.6) (layer "F.Cu") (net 5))
 (segment (start 169.875 90.1) (end 169.875 93.0375) (width 0.6) (layer "F.Cu") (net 5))
 (segment (start 170.0375 95.205002) (end 169.592502 95.65) (width 0.6) (layer "F.Cu") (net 5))
 (segment (start 148.6 84.1) (end 148.4 83.9) (width 0.6) (layer "F.Cu") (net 5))
 (segment (start 148.6 86.605) (end 147.694296 86.605) (width 0.6) (layer "F.Cu") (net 5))
 (segment (start 144.1 90.199296) (end 144.1 92.850002) (width 0.6) (layer "F.Cu") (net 5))
 (segment (start 174.344992 93.2) (end 176.851474 95.706482) (width 0.6) (layer "F.Cu") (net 5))
 (segment (start 148.6 86.605) (end 148.6 84.1) (width 0.6) (layer "F.Cu") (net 5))
 (segment (start 169.85 90.075) (end 169.875 90.1) (width 0.6) (layer "F.Cu") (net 5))
 (segment (start 168.9 94.65) (end 169.9375 94.65) (width 0.6) (layer "F.Cu") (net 5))
 (segment (start 169.442502 97.756482) (end 169.6 97.598984) (width 0.6) (layer "F.Cu") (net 5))
 (segment (start 147.694296 86.605) (end 144.1 90.199296) (width 0.6) (layer "F.Cu") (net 5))
 (segment (start 169.6 97.598984) (end 169.6 95.657498) (width 0.6) (layer "F.Cu") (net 5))
 (segment (start 159.6 98.15) (end 159.6 95.35) (width 0.6) (layer "F.Cu") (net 5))
 (segment (start 170.0375 93.2) (end 174.344992 93.2) (width 0.6) (layer "F.Cu") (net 5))
 (segment (start 169.6 95.657498) (end 169.592502 95.65) (width 0.6) (layer "F.Cu") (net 5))
 (via (at 168.9 94.65) (size 0.7) (drill 0.3) (layers "F.Cu" "B.Cu") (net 5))
 (via (at 144.1 92.850002) (size 0.7) (drill 0.3) (layers "F.Cu" "B.Cu") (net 5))
 (via (at 159.6 95.35) (size 0.7) (drill 0.3) (layers "F.Cu" "B.Cu") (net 5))
 (segment (start 157.1 92.85) (end 159.6 95.35) (width 0.6) (layer "B.Cu") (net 5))
 (segment (start 144.1 92.85) (end 144.1 92.850002) (width 0.6) (layer "B.Cu") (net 5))
 (segment (start 128.03 92.85) (end 144.1 92.85) (width 0.6) (layer "B.Cu") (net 5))
 (segment (start 168.2 95.35) (end 168.9 94.65) (width 0.6) (layer "B.Cu") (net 5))
 (segment (start 144.1 92.85) (end 157.1 92.85) (width 0.6) (layer "B.Cu") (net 5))
 (segment (start 122.16 98.72) (end 128.03 92.85) (width 0.6) (layer "B.Cu") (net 5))
 (segment (start 159.6 95.35) (end 168.2 95.35) (width 0.6) (layer "B.Cu") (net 5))
 (segment (start 164.95 95.45) (end 163.05 93.55) (width 0.6) (layer "F.Cu") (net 13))
 (segment (start 154.55 83.9) (end 155.75 82.7) (width 0.6) (layer "F.Cu") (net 13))
 (segment (start 155.75 82.7) (end 157.6 82.7) (width 0.6) (layer "F.Cu") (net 13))
 (segment (start 164.9 85.1) (end 160 85.1) (width 0.6) (layer "F.Cu") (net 13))
 (segment (start 121.149501 100.249501) (end 162.150499 100.249501) (width 0.6) (layer "F.Cu") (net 13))
 (segment (start 165.925 86.125) (end 164.9 85.1) (width 0.6) (layer "F.Cu") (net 13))
 (segment (start 163.05 93.55) (end 165.925 90.675) (width 0.6) (layer "F.Cu") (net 13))
 (segment (start 119.62 98.72) (end 121.149501 100.249501) (width 0.6) (layer "F.Cu") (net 13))
 (segment (start 157.6 82.7) (end 158.8 83.9) (width 0.6) (layer "F.Cu") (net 13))
 (segment (start 160 85.1) (end 158.8 83.9) (width 0.6) (layer "F.Cu") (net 13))
 (segment (start 165.925 90.675) (end 165.925 86.125) (width 0.6) (layer "F.Cu") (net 13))
 (segment (start 164.95 97.45) (end 164.95 95.45) (width 0.6) (layer "F.Cu") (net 13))
 (segment (start 162.150499 100.249501) (end 164.95 97.45) (width 0.6) (layer "F.Cu") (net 13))
 (segment (start 147.417713 90.415) (end 146.882713 90.95) (width 0.6) (layer "F.Cu") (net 6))
 (segment (start 161.05 83.9) (end 161.05 83.5) (width 0.6) (layer "F.Cu") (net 6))
 (segment (start 147.554962 87.875) (end 148.6 87.875) (width 0.6) (layer "F.Cu") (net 6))
 (segment (start 161.05 83.5) (end 160.2 82.65) (width 0.6) (layer "F.Cu") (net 6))
 (segment (start 149.274239 87.875) (end 150.55 86.599239) (width 0.6) (layer "F.Cu") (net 6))
 (segment (start 145.7 90.95) (end 145.3755 90.6255) (width 0.6) (layer "F.Cu") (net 6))
 (segment (start 148.6 87.875) (end 149.274239 87.875) (width 0.6) (layer "F.Cu") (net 6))
 (segment (start 148.6 90.415) (end 147.417713 90.415) (width 0.6) (layer "F.Cu") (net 6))
 (segment (start 150.55 86.599239) (end 150.55 86) (width 0.6) (layer "F.Cu") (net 6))
 (segment (start 145.3755 90.6255) (end 145.3755 90.054462) (width 0.6) (layer "F.Cu") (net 6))
 (segment (start 146.882713 90.95) (end 145.7 90.95) (width 0.6) (layer "F.Cu") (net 6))
 (segment (start 145.3755 90.054462) (end 147.554962 87.875) (width 0.6) (layer "F.Cu") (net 6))
 (via (at 145.7 90.95) (size 0.7) (drill 0.3) (layers "F.Cu" "B.Cu") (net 6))
 (via (at 150.55 86) (size 0.7) (drill 0.3) (layers "F.Cu" "B.Cu") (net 6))
 (via (at 160.2 82.65) (size 0.7) (drill 0.3) (layers "F.Cu" "B.Cu") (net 6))
 (segment (start 154.8 83.9) (end 154.8 82.95) (width 0.6) (layer "B.Cu") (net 6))
 (segment (start 151.4 82.95) (end 151.7 82.65) (width 0.6) (layer "B.Cu") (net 6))
 (segment (start 154.8 83.15) (end 154.8 83.9) (width 0.6) (layer "B.Cu") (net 6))
 (segment (start 155.1 82.65) (end 160.2 82.65) (width 0.6) (layer "B.Cu") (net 6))
 (segment (start 151.4 83.9) (end 151.4 82.95) (width 0.6) (layer "B.Cu") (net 6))
 (segment (start 151.7 82.65) (end 154.3 82.65) (width 0.6) (layer "B.Cu") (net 6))
 (segment (start 154.8 82.95) (end 155.1 82.65) (width 0.6) (layer "B.Cu") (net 6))
 (segment (start 124.85 90.95) (end 145.7 90.95) (width 0.6) (layer "B.Cu") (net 6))
 (segment (start 154.3 82.65) (end 154.8 83.15) (width 0.6) (layer "B.Cu") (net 6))
 (segment (start 150.55 86) (end 150.55 84.75) (width 0.6) (layer "B.Cu") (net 6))
 (segment (start 117.08 98.72) (end 124.85 90.95) (width 0.6) (layer "B.Cu") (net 6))
 (segment (start 150.55 84.75) (end 151.4 83.9) (width 0.6) (layer "B.Cu") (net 6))
 (segment (start 167.692502 95.8) (end 167.542502 95.65) (width 0.6) (layer "F.Cu") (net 7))
 (segment (start 163.05 83.9) (end 166.16 83.9) (width 0.6) (layer "F.Cu") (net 7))
 (segment (start 167.335002 90.074998) (end 167.335002 85) (width 0.6) (layer "F.Cu") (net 7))
 (segment (start 174.144992 83.6) (end 168.735002 83.6) (width 0.6) (layer "F.Cu") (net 7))
 (segment (start 167.692502 97.756482) (end 167.692502 95.8) (width 0.6) (layer "F.Cu") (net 7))
 (segment (start 147.486338 89.145) (end 146.897606 89.733732) (width 0.6) (layer "F.Cu") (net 7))
 (segment (start 166.16 83.9) (end 167.31 85.05) (width 0.6) (layer "F.Cu") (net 7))
 (segment (start 168.735002 83.6) (end 167.335002 85) (width 0.6) (layer "F.Cu") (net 7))
 (segment (start 167.080002 93.056482) (end 167.080002 90.329998) (width 0.6) (layer "F.Cu") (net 7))
 (segment (start 167.080002 90.329998) (end 167.335002 90.074998) (width 0.6) (layer "F.Cu") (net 7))
 (segment (start 167.542502 95.65) (end 167.542502 93.518982) (width 0.6) (layer "F.Cu") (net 7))
 (segment (start 167.542502 93.518982) (end 167.080002 93.056482) (width 0.6) (layer "F.Cu") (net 7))
 (segment (start 176.851474 86.306482) (end 174.144992 83.6) (width 0.6) (layer "F.Cu") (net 7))
 (segment (start 148.6 89.145) (end 147.486338 89.145) (width 0.6) (layer "F.Cu") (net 7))
 (via (at 146.897606 89.733732) (size 0.7) (drill 0.3) (layers "F.Cu" "B.Cu") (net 7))
 (segment (start 167.31 90.1) (end 163.76 93.65) (width 0.6) (layer "B.Cu") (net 7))
 (segment (start 163.76 93.65) (end 159.65 93.65) (width 0.6) (layer "B.Cu") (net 7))
 (segment (start 123.526268 89.733732) (end 146.897606 89.733732) (width 0.6) (layer "B.Cu") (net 7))
 (segment (start 159.65 93.65) (end 155.733732 89.733732) (width 0.6) (layer "B.Cu") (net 7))
 (segment (start 114.54 98.72) (end 123.526268 89.733732) (width 0.6) (layer "B.Cu") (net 7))
 (segment (start 155.733732 89.733732) (end 146.897606 89.733732) (width 0.6) (layer "B.Cu") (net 7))
 (segment (start 157.9 94.225) (end 156.044334 94.225) (width 0.6) (layer "F.Cu") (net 2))
 (segment (start 154.770333 95.499001) (end 153.75 95.499001) (width 0.6) (layer "F.Cu") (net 2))
 (segment (start 152.700999 95.499001) (end 153.75 95.499001) (width 0.6) (layer "F.Cu") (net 2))
 (segment (start 150 98.1) (end 150.1 98.1) (width 0.6) (layer "F.Cu") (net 2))
 (segment (start 156.044334 94.225) (end 154.770333 95.499001) (width 0.6) (layer "F.Cu") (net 2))
 (segment (start 150.1 98.1) (end 152.700999 95.499001) (width 0.6) (layer "F.Cu") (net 2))
 (via (at 153.75 95.499001) (size 0.7) (drill 0.3) (layers "F.Cu" "B.Cu") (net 2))
 (segment (start 130.460999 95.499001) (end 153.75 95.499001) (width 0.6) (layer "B.Cu") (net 2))
 (segment (start 127.24 98.72) (end 130.460999 95.499001) (width 0.6) (layer "B.Cu") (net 2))
 (segment (start 157.9 95.495) (end 156.356376 95.495) (width 0.6) (layer "F.Cu") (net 9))
 (segment (start 156.356376 95.495) (end 156.300688 95.550688) (width 0.6) (layer "F.Cu") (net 9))
 (segment (start 154.85 97.001376) (end 156.300688 95.550688) (width 0.6) (layer "F.Cu") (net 9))
 (segment (start 154.85 98.15) (end 154.85 97.001376) (width 0.6) (layer "F.Cu") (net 9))
 (via (at 156.300688 95.550688) (size 0.7) (drill 0.3) (layers "F.Cu" "B.Cu") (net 9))
 (segment (start 154.8 94.05) (end 156.300688 95.550688) (width 0.6) (layer "B.Cu") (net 9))
 (segment (start 129.37 94.05) (end 154.8 94.05) (width 0.6) (layer "B.Cu") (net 9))
 (segment (start 124.7 98.72) (end 129.37 94.05) (width 0.6) (layer "B.Cu") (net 9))
 (segment (start 161.05 91.2) (end 160.05 91.2) (width 0.6) (layer "F.Cu") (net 4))
 (via (at 160.05 91.2) (size 0.7) (drill 0.3) (layers "F.Cu" "B.Cu") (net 4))
 (segment (start 106.92 98.72) (end 117.29 88.35) (width 0.6) (layer "B.Cu") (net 4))
 (segment (start 117.29 88.35) (end 157.2 88.35) (width 0.6) (layer "B.Cu") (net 4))
 (segment (start 157.2 88.35) (end 160.05 91.2) (width 0.6) (layer "B.Cu") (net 4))
 (segment (start 131.13 82.13) (end 129.78 83.48) (width 0.6) (layer "F.Cu") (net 20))
 (segment (start 152.55 83.9) (end 150.78 82.13) (width 0.6) (layer "F.Cu") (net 20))
 (segment (start 150.78 82.13) (end 131.13 82.13) (width 0.6) (layer "F.Cu") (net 20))
 (segment (start 161.05 93.5) (end 162.1 92.45) (width 0.6) (layer "F.Cu") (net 28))
 (segment (start 161.05 93.55) (end 161.05 93.5) (width 0.6) (layer "F.Cu") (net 28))
 (via (at 162.1 92.45) (size 0.7) (drill 0.3) (layers "F.Cu" "B.Cu") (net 28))
 (segment (start 113.13 87.15) (end 109.46 83.48) (width 0.6) (layer "B.Cu") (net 28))
 (segment (start 162.1 90.85) (end 158.4 87.15) (width 0.6) (layer "B.Cu") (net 28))
 (segment (start 162.1 92.45) (end 162.1 90.85) (width 0.6) (layer "B.Cu") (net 28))
 (segment (start 158.4 87.15) (end 113.13 87.15) (width 0.6) (layer "B.Cu") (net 28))
 (segment (start 164.55 87.775) (end 163.075 86.3) (width 0.6) (layer "F.Cu") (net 3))
 (segment (start 164.55 89.7) (end 164.55 87.775) (width 0.6) (layer "F.Cu") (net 3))
 (segment (start 163.05 91.2) (end 164.55 89.7) (width 0.6) (layer "F.Cu") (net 3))
 (segment (start 156.905 92.955) (end 155.399999 91.449999) (width 0.6) (layer "F.Cu") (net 10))
 (segment (start 157.9 92.955) (end 156.905 92.955) (width 0.6) (layer "F.Cu") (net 10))
 (via (at 155.399999 91.449999) (size 0.7) (drill 0.3) (layers "F.Cu" "B.Cu") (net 10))
 (segment (start 151.3 91.45) (end 155.399999 91.449999) (width 0.6) (layer "B.Cu") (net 10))
 (segment (start 155.675 87.875) (end 153.55 85.75) (width 0.6) (layer "F.Cu") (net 11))
 (segment (start 157.9 87.875) (end 155.675 87.875) (width 0.6) (layer "F.Cu") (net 11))
 (via (at 153.55 85.75) (size 0.7) (drill 0.3) (layers "F.Cu" "B.Cu") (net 11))
 (segment (start 152.7 84.9) (end 153.55 85.75) (width 0.6) (layer "B.Cu") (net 11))
 (segment (start 152.7 83.9) (end 152.7 84.9) (width 0.6) (layer "B.Cu") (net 11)))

